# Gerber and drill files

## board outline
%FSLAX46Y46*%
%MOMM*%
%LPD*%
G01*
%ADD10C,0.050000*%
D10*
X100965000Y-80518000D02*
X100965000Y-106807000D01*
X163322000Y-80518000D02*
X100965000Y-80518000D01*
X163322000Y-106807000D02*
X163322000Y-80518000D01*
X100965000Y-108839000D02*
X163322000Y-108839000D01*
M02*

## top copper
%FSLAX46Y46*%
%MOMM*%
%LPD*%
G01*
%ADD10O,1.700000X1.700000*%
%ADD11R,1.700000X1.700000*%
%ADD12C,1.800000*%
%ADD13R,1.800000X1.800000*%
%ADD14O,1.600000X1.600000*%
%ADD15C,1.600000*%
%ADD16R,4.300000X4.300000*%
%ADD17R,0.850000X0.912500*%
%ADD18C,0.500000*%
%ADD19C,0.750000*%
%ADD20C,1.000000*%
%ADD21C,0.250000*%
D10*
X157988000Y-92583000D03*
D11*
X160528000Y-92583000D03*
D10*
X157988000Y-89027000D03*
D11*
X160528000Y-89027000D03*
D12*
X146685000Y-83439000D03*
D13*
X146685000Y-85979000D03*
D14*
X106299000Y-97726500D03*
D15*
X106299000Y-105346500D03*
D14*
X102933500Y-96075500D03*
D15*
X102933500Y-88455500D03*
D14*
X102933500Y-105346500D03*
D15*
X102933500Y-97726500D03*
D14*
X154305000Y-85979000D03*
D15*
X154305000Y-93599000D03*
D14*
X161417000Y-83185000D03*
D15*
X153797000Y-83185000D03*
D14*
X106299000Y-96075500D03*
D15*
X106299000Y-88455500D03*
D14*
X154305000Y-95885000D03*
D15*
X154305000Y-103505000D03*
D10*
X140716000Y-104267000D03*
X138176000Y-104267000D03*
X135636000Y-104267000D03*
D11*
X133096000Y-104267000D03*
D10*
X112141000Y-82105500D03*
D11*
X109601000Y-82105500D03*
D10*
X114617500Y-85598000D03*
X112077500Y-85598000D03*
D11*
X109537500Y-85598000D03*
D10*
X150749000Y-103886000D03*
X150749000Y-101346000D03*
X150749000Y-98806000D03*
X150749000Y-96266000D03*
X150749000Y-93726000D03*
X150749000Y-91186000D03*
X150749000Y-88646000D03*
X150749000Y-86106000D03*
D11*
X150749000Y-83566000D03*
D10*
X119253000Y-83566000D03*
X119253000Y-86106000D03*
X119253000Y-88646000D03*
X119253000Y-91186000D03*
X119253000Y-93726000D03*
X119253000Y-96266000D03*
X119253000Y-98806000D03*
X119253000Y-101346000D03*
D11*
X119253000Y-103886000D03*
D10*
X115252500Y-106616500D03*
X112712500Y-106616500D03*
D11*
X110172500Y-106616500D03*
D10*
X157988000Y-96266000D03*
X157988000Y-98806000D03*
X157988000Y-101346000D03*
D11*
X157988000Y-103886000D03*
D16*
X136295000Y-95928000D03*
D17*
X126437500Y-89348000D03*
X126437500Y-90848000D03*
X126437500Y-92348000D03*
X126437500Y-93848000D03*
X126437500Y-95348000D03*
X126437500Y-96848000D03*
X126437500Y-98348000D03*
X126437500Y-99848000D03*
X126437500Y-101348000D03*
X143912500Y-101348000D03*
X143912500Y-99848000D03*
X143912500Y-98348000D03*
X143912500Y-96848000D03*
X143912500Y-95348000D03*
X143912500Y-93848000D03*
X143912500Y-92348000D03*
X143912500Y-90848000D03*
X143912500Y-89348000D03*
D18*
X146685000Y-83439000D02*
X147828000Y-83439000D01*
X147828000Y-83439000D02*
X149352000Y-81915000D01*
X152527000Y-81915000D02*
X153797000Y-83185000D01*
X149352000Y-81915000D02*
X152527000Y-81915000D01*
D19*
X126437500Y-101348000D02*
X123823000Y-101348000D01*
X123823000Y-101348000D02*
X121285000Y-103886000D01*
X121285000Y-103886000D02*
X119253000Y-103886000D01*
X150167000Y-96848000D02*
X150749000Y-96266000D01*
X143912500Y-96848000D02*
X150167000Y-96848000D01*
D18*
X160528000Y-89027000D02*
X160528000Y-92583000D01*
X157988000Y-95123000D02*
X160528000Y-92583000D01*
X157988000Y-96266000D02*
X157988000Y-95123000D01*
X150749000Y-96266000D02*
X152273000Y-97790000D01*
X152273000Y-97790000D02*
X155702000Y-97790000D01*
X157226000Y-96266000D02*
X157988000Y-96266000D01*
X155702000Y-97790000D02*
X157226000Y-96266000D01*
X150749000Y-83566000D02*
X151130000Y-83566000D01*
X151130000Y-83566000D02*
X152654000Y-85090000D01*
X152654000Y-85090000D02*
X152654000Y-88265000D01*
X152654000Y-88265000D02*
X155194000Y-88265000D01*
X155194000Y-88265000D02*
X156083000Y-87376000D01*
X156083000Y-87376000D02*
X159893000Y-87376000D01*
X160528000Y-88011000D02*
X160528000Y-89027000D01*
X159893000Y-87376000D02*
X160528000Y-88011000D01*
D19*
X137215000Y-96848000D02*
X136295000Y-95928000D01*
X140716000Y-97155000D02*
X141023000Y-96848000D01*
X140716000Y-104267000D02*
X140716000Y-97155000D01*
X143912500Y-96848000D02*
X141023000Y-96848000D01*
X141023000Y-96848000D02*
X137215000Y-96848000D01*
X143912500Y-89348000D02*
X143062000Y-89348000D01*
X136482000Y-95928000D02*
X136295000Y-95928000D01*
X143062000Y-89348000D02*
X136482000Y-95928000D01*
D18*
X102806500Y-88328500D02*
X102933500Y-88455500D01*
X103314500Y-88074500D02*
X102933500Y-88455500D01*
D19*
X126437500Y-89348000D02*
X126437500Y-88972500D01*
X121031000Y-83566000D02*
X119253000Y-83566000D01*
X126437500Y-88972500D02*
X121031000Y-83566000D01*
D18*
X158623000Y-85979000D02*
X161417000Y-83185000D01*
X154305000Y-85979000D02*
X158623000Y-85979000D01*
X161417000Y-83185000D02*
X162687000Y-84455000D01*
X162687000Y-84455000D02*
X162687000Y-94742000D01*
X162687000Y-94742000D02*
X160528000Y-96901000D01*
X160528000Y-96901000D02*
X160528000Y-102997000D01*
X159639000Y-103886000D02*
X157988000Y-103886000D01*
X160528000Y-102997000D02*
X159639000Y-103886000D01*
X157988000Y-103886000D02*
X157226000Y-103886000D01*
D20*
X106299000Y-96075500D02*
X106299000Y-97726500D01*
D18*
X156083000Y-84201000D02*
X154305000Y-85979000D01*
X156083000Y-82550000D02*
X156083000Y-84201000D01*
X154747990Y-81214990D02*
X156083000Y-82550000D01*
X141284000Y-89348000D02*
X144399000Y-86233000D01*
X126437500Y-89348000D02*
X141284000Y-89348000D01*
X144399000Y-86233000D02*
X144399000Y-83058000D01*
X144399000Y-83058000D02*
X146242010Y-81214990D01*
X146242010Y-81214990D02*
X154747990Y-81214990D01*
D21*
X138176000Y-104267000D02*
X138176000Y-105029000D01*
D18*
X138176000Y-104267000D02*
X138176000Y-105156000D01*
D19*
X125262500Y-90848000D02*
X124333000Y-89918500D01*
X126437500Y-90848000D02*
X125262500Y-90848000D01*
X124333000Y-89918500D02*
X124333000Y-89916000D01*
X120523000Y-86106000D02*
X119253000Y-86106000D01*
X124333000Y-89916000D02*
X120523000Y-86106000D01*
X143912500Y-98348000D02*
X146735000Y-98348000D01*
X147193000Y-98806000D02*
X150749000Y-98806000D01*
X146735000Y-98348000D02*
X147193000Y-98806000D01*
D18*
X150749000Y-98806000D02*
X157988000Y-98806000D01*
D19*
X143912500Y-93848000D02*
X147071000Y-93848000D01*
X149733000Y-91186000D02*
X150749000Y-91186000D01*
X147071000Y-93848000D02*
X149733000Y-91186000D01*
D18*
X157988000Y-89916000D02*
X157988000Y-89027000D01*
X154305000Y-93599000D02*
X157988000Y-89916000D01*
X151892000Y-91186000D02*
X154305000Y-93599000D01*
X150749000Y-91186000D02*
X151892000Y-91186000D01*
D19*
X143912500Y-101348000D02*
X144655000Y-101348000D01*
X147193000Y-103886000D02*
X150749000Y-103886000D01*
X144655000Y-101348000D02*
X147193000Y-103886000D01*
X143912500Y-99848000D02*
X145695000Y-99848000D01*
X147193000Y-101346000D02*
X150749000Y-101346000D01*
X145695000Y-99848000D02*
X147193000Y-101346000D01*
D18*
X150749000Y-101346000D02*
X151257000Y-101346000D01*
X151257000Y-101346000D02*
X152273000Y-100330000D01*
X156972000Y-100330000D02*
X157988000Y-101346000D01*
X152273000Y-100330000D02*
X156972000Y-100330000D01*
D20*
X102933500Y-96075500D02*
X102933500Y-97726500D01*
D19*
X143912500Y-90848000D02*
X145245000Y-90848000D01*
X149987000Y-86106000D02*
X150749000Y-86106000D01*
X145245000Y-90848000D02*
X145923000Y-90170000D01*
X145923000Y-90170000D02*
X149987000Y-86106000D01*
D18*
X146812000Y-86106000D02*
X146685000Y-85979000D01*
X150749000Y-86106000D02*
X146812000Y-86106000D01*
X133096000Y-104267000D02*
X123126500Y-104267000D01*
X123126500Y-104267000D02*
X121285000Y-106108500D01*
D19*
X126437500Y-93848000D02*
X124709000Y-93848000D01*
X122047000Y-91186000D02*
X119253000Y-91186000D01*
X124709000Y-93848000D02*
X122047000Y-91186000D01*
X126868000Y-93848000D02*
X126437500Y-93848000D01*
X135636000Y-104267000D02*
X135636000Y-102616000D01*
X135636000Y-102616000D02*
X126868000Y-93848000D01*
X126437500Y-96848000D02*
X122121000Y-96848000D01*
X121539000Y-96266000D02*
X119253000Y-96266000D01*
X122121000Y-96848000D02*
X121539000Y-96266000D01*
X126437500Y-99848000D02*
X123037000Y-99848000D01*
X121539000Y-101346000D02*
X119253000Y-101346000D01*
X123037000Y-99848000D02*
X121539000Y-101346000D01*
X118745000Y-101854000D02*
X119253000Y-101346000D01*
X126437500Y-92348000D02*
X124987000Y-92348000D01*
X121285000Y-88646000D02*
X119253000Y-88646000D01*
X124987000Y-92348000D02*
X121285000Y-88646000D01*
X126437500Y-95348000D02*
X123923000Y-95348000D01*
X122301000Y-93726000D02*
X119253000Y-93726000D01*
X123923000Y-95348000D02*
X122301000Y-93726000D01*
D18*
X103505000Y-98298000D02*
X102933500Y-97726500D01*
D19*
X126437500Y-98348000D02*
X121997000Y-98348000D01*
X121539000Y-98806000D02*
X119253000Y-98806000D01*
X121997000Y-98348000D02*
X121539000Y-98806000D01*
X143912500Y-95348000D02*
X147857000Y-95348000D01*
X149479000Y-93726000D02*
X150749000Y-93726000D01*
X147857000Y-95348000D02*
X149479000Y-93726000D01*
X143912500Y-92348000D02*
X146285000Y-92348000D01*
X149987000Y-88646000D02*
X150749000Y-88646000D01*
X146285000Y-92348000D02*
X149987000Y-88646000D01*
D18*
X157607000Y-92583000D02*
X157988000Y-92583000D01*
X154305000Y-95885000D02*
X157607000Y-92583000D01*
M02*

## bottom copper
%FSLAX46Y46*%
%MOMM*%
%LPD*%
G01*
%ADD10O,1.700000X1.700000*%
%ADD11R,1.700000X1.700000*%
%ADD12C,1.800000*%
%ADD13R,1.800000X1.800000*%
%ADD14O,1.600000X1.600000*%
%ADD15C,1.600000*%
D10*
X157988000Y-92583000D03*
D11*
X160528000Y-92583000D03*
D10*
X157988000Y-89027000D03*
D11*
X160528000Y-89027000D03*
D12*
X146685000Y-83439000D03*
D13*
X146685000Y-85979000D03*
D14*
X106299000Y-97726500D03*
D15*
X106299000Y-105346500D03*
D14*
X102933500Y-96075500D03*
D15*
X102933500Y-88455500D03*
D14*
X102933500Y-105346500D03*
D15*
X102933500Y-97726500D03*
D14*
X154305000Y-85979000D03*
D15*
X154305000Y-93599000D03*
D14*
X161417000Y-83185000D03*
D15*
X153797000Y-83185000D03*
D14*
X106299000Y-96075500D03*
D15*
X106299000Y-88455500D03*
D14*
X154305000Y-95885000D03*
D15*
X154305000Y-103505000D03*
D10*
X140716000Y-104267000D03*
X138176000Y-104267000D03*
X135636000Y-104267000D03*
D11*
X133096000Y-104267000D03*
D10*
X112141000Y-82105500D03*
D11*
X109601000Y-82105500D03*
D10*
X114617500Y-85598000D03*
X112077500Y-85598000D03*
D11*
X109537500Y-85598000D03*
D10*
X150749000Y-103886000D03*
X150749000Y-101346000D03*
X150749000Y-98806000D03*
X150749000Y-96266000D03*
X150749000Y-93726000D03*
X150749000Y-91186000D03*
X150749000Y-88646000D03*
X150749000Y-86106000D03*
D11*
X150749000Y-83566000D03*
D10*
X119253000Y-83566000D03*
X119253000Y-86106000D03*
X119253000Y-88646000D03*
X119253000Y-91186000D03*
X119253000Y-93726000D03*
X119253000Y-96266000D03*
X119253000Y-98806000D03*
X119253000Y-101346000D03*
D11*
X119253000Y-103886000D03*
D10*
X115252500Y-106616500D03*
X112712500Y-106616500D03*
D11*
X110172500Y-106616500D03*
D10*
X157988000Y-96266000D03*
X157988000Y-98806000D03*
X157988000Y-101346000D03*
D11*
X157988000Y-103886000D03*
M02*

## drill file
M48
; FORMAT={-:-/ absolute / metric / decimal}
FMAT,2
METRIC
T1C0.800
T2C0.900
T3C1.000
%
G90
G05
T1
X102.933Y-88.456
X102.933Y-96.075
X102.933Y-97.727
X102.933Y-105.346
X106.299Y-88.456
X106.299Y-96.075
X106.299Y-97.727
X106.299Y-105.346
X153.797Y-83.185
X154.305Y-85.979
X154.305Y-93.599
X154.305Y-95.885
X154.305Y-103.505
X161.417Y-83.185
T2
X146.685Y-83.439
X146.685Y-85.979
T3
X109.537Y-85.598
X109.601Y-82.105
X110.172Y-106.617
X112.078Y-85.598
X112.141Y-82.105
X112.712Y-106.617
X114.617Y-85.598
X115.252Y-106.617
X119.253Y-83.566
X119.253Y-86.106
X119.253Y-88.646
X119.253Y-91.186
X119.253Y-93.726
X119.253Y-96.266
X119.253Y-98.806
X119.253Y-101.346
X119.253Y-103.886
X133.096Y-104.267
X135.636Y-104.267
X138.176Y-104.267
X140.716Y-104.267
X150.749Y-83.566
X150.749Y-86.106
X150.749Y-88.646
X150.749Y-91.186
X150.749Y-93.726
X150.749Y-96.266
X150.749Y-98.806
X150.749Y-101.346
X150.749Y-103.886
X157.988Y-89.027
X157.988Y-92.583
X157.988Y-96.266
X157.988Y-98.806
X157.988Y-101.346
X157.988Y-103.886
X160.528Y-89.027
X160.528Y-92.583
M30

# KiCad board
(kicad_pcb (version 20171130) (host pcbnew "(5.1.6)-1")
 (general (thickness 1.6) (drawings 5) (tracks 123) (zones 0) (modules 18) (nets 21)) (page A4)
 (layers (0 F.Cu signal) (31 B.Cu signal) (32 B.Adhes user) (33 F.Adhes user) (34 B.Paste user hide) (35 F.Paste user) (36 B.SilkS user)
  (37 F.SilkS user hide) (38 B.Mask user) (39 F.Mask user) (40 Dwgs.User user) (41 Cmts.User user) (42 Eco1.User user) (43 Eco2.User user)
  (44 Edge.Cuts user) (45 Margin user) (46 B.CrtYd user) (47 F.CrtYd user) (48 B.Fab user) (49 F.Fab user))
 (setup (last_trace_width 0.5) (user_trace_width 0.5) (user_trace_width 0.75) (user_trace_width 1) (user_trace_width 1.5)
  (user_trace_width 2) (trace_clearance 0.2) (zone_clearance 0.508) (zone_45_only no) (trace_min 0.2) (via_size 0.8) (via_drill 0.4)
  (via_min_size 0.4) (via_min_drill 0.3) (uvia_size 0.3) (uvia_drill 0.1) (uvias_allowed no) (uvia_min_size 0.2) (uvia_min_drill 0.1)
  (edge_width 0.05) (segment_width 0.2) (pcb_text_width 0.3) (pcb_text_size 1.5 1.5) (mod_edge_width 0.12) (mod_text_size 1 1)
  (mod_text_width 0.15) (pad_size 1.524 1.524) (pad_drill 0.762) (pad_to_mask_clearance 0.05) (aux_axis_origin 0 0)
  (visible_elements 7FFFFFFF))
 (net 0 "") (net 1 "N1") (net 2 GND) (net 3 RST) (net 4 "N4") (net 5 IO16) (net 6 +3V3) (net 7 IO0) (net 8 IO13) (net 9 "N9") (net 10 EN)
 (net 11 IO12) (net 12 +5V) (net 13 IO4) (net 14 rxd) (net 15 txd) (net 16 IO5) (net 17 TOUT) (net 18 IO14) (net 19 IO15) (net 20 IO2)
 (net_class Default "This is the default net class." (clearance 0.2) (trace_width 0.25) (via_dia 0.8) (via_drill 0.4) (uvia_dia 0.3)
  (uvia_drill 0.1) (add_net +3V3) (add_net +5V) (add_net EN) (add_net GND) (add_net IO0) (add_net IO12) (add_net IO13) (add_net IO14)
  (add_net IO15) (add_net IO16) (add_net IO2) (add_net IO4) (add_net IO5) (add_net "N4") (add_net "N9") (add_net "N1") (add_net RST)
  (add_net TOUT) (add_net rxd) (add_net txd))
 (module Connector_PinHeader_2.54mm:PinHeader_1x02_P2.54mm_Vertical (layer F.Cu) (at 160.528 92.583 270)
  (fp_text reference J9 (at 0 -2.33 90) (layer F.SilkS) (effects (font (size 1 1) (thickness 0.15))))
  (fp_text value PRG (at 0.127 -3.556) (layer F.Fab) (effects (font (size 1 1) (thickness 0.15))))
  (pad 2 thru_hole oval (at 0 2.54 270) (size 1.7 1.7) (drill 1) (layers *.Cu *.Mask) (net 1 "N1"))
  (pad 1 thru_hole rect (at 0 0 270) (size 1.7 1.7) (drill 1) (layers *.Cu *.Mask) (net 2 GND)))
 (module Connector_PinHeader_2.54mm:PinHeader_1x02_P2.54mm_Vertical (layer F.Cu) (at 160.528 89.027 270)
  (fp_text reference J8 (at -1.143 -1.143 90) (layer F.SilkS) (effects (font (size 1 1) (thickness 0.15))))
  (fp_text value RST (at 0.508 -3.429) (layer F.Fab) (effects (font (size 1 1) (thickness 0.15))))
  (pad 2 thru_hole oval (at 0 2.54 270) (size 1.7 1.7) (drill 1) (layers *.Cu *.Mask) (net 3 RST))
  (pad 1 thru_hole rect (at 0 0 270) (size 1.7 1.7) (drill 1) (layers *.Cu *.Mask) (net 2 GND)))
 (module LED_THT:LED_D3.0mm (layer F.Cu) (at 146.685 85.979 90)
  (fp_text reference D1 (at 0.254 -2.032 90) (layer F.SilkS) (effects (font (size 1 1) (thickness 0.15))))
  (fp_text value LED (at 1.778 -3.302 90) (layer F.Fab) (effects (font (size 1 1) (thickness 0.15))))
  (pad 2 thru_hole circle (at 2.54 0 90) (size 1.8 1.8) (drill 0.9) (layers *.Cu *.Mask) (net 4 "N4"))
  (pad 1 thru_hole rect (at 0 0 90) (size 1.8 1.8) (drill 0.9) (layers *.Cu *.Mask) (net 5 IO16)))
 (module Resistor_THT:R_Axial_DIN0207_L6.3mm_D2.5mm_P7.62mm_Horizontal (layer F.Cu) (at 106.299 105.3465 90)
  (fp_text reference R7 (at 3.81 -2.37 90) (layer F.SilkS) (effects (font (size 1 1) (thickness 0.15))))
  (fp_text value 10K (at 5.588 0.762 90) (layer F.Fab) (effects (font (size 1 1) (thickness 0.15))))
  (pad 2 thru_hole oval (at 7.62 0 90) (size 1.6 1.6) (drill 0.8) (layers *.Cu *.Mask) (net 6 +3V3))
  (pad 1 thru_hole circle (at 0 0 90) (size 1.6 1.6) (drill 0.8) (layers *.Cu *.Mask) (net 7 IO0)))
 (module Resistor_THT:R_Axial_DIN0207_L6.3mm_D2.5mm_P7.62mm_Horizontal (layer F.Cu) (at 102.9335 88.4555 270)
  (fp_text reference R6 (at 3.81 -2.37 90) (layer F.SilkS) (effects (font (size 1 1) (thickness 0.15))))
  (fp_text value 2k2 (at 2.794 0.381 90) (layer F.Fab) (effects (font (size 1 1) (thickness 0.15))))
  (pad 2 thru_hole oval (at 7.62 0 270) (size 1.6 1.6) (drill 0.8) (layers *.Cu *.Mask) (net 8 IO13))
  (pad 1 thru_hole circle (at 0 0 270) (size 1.6 1.6) (drill 0.8) (layers *.Cu *.Mask) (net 2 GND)))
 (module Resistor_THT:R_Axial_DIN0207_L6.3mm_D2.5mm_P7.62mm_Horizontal (layer F.Cu) (at 102.9335 97.7265 270)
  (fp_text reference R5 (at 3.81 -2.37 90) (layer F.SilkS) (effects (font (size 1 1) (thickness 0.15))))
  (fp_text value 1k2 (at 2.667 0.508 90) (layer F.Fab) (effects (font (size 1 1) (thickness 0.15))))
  (pad 2 thru_hole oval (at 7.62 0 270) (size 1.6 1.6) (drill 0.8) (layers *.Cu *.Mask) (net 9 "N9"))
  (pad 1 thru_hole circle (at 0 0 270) (size 1.6 1.6) (drill 0.8) (layers *.Cu *.Mask) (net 8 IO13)))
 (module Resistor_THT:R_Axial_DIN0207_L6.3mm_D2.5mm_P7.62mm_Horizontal (layer F.Cu) (at 154.305 93.599 90)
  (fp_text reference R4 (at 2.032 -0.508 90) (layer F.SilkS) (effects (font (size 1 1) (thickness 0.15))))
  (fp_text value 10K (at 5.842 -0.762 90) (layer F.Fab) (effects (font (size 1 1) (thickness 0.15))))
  (pad 2 thru_hole oval (at 7.62 0 90) (size 1.6 1.6) (drill 0.8) (layers *.Cu *.Mask) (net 6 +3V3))
  (pad 1 thru_hole circle (at 0 0 90) (size 1.6 1.6) (drill 0.8) (layers *.Cu *.Mask) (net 3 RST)))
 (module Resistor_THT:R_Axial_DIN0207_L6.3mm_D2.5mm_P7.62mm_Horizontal (layer F.Cu) (at 153.797 83.185)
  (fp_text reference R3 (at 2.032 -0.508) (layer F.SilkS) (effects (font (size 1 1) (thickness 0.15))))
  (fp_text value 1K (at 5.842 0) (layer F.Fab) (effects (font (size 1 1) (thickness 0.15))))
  (pad 2 thru_hole oval (at 7.62 0) (size 1.6 1.6) (drill 0.8) (layers *.Cu *.Mask) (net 6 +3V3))
  (pad 1 thru_hole circle (at 0 0) (size 1.6 1.6) (drill 0.8) (layers *.Cu *.Mask) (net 4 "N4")))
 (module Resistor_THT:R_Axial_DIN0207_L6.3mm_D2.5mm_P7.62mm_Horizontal (layer F.Cu) (at 106.299 88.4555 270)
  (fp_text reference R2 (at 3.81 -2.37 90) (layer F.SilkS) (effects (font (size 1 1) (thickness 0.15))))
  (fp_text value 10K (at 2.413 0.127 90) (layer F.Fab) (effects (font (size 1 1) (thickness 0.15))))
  (pad 2 thru_hole oval (at 7.62 0 270) (size 1.6 1.6) (drill 0.8) (layers *.Cu *.Mask) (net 6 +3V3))
  (pad 1 thru_hole circle (at 0 0 270) (size 1.6 1.6) (drill 0.8) (layers *.Cu *.Mask) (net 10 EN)))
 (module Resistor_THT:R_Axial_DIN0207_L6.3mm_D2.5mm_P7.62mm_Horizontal (layer F.Cu) (at 154.305 103.505 90)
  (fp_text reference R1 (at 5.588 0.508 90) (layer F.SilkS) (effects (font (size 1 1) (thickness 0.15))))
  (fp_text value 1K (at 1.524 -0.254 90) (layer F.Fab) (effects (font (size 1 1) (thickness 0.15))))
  (pad 2 thru_hole oval (at 7.62 0 90) (size 1.6 1.6) (drill 0.8) (layers *.Cu *.Mask) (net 1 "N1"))
  (pad 1 thru_hole circle (at 0 0 90) (size 1.6 1.6) (drill 0.8) (layers *.Cu *.Mask) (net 7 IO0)))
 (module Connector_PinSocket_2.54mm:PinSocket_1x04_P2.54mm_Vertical (layer F.Cu) (at 133.096 104.267 90)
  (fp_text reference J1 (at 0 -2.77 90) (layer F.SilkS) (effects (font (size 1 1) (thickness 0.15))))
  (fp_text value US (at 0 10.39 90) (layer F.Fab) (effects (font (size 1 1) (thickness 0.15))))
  (pad 4 thru_hole oval (at 0 7.62 90) (size 1.7 1.7) (drill 1) (layers *.Cu *.Mask) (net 2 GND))
  (pad 3 thru_hole oval (at 0 5.08 90) (size 1.7 1.7) (drill 1) (layers *.Cu *.Mask) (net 9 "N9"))
  (pad 2 thru_hole oval (at 0 2.54 90) (size 1.7 1.7) (drill 1) (layers *.Cu *.Mask) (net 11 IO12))
  (pad 1 thru_hole rect (at 0 0 90) (size 1.7 1.7) (drill 1) (layers *.Cu *.Mask) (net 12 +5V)))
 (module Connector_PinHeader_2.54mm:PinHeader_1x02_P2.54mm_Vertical (layer F.Cu) (at 109.601 82.1055 90)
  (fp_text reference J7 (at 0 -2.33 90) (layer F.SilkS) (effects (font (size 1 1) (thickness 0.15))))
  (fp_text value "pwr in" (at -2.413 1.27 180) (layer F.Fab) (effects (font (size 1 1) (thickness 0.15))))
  (pad 2 thru_hole oval (at 0 2.54 90) (size 1.7 1.7) (drill 1) (layers *.Cu *.Mask) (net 2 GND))
  (pad 1 thru_hole rect (at 0 0 90) (size 1.7 1.7) (drill 1) (layers *.Cu *.Mask) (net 12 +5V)))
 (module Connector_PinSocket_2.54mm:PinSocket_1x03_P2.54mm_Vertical (layer F.Cu) (at 109.5375 85.598 90)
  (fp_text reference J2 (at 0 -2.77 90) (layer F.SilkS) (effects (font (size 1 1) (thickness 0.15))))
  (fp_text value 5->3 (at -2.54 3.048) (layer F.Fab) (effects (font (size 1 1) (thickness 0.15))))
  (pad 3 thru_hole oval (at 0 5.08 90) (size 1.7 1.7) (drill 1) (layers *.Cu *.Mask) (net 2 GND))
  (pad 2 thru_hole oval (at 0 2.54 90) (size 1.7 1.7) (drill 1) (layers *.Cu *.Mask) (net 6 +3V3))
  (pad 1 thru_hole rect (at 0 0 90) (size 1.7 1.7) (drill 1) (layers *.Cu *.Mask) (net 12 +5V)))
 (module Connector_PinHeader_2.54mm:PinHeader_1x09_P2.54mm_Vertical (layer F.Cu) (at 150.749 83.566)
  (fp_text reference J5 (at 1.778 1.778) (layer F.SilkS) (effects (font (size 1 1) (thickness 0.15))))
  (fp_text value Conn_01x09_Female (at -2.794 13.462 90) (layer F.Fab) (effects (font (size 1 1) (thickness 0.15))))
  (pad 9 thru_hole oval (at 0 20.32) (size 1.7 1.7) (drill 1) (layers *.Cu *.Mask) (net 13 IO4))
  (pad 8 thru_hole oval (at 0 17.78) (size 1.7 1.7) (drill 1) (layers *.Cu *.Mask) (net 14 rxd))
  (pad 7 thru_hole oval (at 0 15.24) (size 1.7 1.7) (drill 1) (layers *.Cu *.Mask) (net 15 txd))
  (pad 6 thru_hole oval (at 0 12.7) (size 1.7 1.7) (drill 1) (layers *.Cu *.Mask) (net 2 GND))
  (pad 5 thru_hole oval (at 0 10.16) (size 1.7 1.7) (drill 1) (layers *.Cu *.Mask) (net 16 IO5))
  (pad 4 thru_hole oval (at 0 7.62) (size 1.7 1.7) (drill 1) (layers *.Cu *.Mask) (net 3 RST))
  (pad 3 thru_hole oval (at 0 5.08) (size 1.7 1.7) (drill 1) (layers *.Cu *.Mask) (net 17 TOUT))
  (pad 2 thru_hole oval (at 0 2.54) (size 1.7 1.7) (drill 1) (layers *.Cu *.Mask) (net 5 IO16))
  (pad 1 thru_hole rect (at 0 0) (size 1.7 1.7) (drill 1) (layers *.Cu *.Mask) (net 2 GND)))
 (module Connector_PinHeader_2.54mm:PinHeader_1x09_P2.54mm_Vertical (layer F.Cu) (at 119.253 103.886 180)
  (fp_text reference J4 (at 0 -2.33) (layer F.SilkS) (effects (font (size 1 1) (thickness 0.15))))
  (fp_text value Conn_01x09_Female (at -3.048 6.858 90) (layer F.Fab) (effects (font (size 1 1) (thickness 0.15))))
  (pad 9 thru_hole oval (at 0 20.32 180) (size 1.7 1.7) (drill 1) (layers *.Cu *.Mask) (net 6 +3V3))
  (pad 8 thru_hole oval (at 0 17.78 180) (size 1.7 1.7) (drill 1) (layers *.Cu *.Mask) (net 10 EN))
  (pad 7 thru_hole oval (at 0 15.24 180) (size 1.7 1.7) (drill 1) (layers *.Cu *.Mask) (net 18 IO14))
  (pad 6 thru_hole oval (at 0 12.7 180) (size 1.7 1.7) (drill 1) (layers *.Cu *.Mask) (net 11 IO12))
  (pad 5 thru_hole oval (at 0 10.16 180) (size 1.7 1.7) (drill 1) (layers *.Cu *.Mask) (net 8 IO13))
  (pad 4 thru_hole oval (at 0 7.62 180) (size 1.7 1.7) (drill 1) (layers *.Cu *.Mask) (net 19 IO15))
  (pad 3 thru_hole oval (at 0 5.08 180) (size 1.7 1.7) (drill 1) (layers *.Cu *.Mask) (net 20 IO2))
  (pad 2 thru_hole oval (at 0 2.54 180) (size 1.7 1.7) (drill 1) (layers *.Cu *.Mask) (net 7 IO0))
  (pad 1 thru_hole rect (at 0 0 180) (size 1.7 1.7) (drill 1) (layers *.Cu *.Mask) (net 2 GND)))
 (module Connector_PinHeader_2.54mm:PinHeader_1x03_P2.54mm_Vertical (layer F.Cu) (at 110.1725 106.6165 90)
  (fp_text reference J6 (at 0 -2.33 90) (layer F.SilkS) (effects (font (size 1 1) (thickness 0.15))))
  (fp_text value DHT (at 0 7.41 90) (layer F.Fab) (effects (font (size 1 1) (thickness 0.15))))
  (pad 3 thru_hole oval (at 0 5.08 90) (size 1.7 1.7) (drill 1) (layers *.Cu *.Mask) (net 18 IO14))
  (pad 2 thru_hole oval (at 0 2.54 90) (size 1.7 1.7) (drill 1) (layers *.Cu *.Mask) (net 2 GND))
  (pad 1 thru_hole rect (at 0 0 90) (size 1.7 1.7) (drill 1) (layers *.Cu *.Mask) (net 6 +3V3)))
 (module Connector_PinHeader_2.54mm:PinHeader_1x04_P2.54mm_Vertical (layer F.Cu) (at 157.988 103.886 180)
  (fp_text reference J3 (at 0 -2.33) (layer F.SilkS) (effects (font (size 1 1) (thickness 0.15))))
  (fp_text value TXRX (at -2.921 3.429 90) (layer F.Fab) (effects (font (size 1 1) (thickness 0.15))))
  (pad 4 thru_hole oval (at 0 7.62 180) (size 1.7 1.7) (drill 1) (layers *.Cu *.Mask) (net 2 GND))
  (pad 3 thru_hole oval (at 0 5.08 180) (size 1.7 1.7) (drill 1) (layers *.Cu *.Mask) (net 15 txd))
  (pad 2 thru_hole oval (at 0 2.54 180) (size 1.7 1.7) (drill 1) (layers *.Cu *.Mask) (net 14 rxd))
  (pad 1 thru_hole rect (at 0 0 180) (size 1.7 1.7) (drill 1) (layers *.Cu *.Mask) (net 6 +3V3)))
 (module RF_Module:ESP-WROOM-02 (layer F.Cu) (at 135.175 95.348)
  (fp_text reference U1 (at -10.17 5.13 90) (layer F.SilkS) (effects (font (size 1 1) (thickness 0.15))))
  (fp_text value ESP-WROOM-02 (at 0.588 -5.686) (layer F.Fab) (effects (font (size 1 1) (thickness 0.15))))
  (pad 19 smd rect (at 1.12 0.58) (size 4.3 4.3) (layers F.Cu F.Paste F.Mask) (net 2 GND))
  (pad 1 smd rect (at -8.7375 -6) (size 0.85 0.9125) (layers F.Cu F.Paste F.Mask) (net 6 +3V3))
  (pad 2 smd rect (at -8.7375 -4.5) (size 0.85 0.9125) (layers F.Cu F.Paste F.Mask) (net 10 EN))
  (pad 3 smd rect (at -8.7375 -3) (size 0.85 0.9125) (layers F.Cu F.Paste F.Mask) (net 18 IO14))
  (pad 4 smd rect (at -8.7375 -1.5) (size 0.85 0.9125) (layers F.Cu F.Paste F.Mask) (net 11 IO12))
  (pad 5 smd rect (at -8.7375 0) (size 0.85 0.9125) (layers F.Cu F.Paste F.Mask) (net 8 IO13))
  (pad 6 smd rect (at -8.7375 1.5) (size 0.85 0.9125) (layers F.Cu F.Paste F.Mask) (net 19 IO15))
  (pad 7 smd rect (at -8.7375 3) (size 0.85 0.9125) (layers F.Cu F.Paste F.Mask) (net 20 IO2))
  (pad 8 smd rect (at -8.7375 4.5) (size 0.85 0.9125) (layers F.Cu F.Paste F.Mask) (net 7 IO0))
  (pad 9 smd rect (at -8.7375 6) (size 0.85 0.9125) (layers F.Cu F.Paste F.Mask) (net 2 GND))
  (pad 10 smd rect (at 8.7375 6) (size 0.85 0.9125) (layers F.Cu F.Paste F.Mask) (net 13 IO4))
  (pad 11 smd rect (at 8.7375 4.5) (size 0.85 0.9125) (layers F.Cu F.Paste F.Mask) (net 14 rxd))
  (pad 12 smd rect (at 8.7375 3) (size 0.85 0.9125) (layers F.Cu F.Paste F.Mask) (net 15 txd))
  (pad 13 smd rect (at 8.7375 1.5) (size 0.85 0.9125) (layers F.Cu F.Paste F.Mask) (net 2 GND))
  (pad 14 smd rect (at 8.7375 0) (size 0.85 0.9125) (layers F.Cu F.Paste F.Mask) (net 16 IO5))
  (pad 15 smd rect (at 8.7375 -1.5) (size 0.85 0.9125) (layers F.Cu F.Paste F.Mask) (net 3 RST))
  (pad 16 smd rect (at 8.7375 -3) (size 0.85 0.9125) (layers F.Cu F.Paste F.Mask) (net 17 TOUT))
  (pad 17 smd rect (at 8.7375 -4.5) (size 0.85 0.9125) (layers F.Cu F.Paste F.Mask) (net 5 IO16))
  (pad 18 smd rect (at 8.7375 -6) (size 0.85 0.9125) (layers F.Cu F.Paste F.Mask) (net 2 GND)))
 (gr_line (start 100.965 80.518) (end 100.965 106.807) (layer Edge.Cuts) (width 0.05))
 (gr_line (start 163.322 80.518) (end 100.965 80.518) (layer Edge.Cuts) (width 0.05))
 (gr_line (start 163.322 106.807) (end 163.322 80.518) (layer Edge.Cuts) (width 0.05))
 (gr_line (start 100.965 108.839) (end 163.322 108.839) (layer Edge.Cuts) (width 0.05))
 (segment (start 146.685 83.439) (end 147.828 83.439) (width 0.5) (layer F.Cu) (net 4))
 (segment (start 147.828 83.439) (end 149.352 81.915) (width 0.5) (layer F.Cu) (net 4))
 (segment (start 152.527 81.915) (end 153.797 83.185) (width 0.5) (layer F.Cu) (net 4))
 (segment (start 149.352 81.915) (end 152.527 81.915) (width 0.5) (layer F.Cu) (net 4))
 (segment (start 126.4375 101.348) (end 123.823 101.348) (width 0.75) (layer F.Cu) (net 2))
 (segment (start 123.823 101.348) (end 121.285 103.886) (width 0.75) (layer F.Cu) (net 2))
 (segment (start 121.285 103.886) (end 119.253 103.886) (width 0.75) (layer F.Cu) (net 2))
 (segment (start 150.167 96.848) (end 150.749 96.266) (width 0.75) (layer F.Cu) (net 2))
 (segment (start 143.9125 96.848) (end 150.167 96.848) (width 0.75) (layer F.Cu) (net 2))
 (segment (start 160.528 89.027) (end 160.528 92.583) (width 0.5) (layer F.Cu) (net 2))
 (segment (start 157.988 95.123) (end 160.528 92.583) (width 0.5) (layer F.Cu) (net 2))
 (segment (start 157.988 96.266) (end 157.988 95.123) (width 0.5) (layer F.Cu) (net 2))
 (segment (start 150.749 96.266) (end 152.273 97.79) (width 0.5) (layer F.Cu) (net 2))
 (segment (start 152.273 97.79) (end 155.702 97.79) (width 0.5) (layer F.Cu) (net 2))
 (segment (start 157.226 96.266) (end 157.988 96.266) (width 0.5) (layer F.Cu) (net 2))
 (segment (start 155.702 97.79) (end 157.226 96.266) (width 0.5) (layer F.Cu) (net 2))
 (segment (start 150.749 83.566) (end 151.13 83.566) (width 0.5) (layer F.Cu) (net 2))
 (segment (start 151.13 83.566) (end 152.654 85.09) (width 0.5) (layer F.Cu) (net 2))
 (segment (start 152.654 85.09) (end 152.654 88.265) (width 0.5) (layer F.Cu) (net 2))
 (segment (start 152.654 88.265) (end 155.194 88.265) (width 0.5) (layer F.Cu) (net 2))
 (segment (start 155.194 88.265) (end 156.083 87.376) (width 0.5) (layer F.Cu) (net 2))
 (segment (start 156.083 87.376) (end 159.893 87.376) (width 0.5) (layer F.Cu) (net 2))
 (segment (start 160.528 88.011) (end 160.528 89.027) (width 0.5) (layer F.Cu) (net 2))
 (segment (start 159.893 87.376) (end 160.528 88.011) (width 0.5) (layer F.Cu) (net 2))
 (segment (start 137.215 96.848) (end 136.295 95.928) (width 0.75) (layer F.Cu) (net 2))
 (segment (start 140.716 97.155) (end 141.023 96.848) (width 0.75) (layer F.Cu) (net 2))
 (segment (start 140.716 104.267) (end 140.716 97.155) (width 0.75) (layer F.Cu) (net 2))
 (segment (start 143.9125 96.848) (end 141.023 96.848) (width 0.75) (layer F.Cu) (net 2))
 (segment (start 141.023 96.848) (end 137.215 96.848) (width 0.75) (layer F.Cu) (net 2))
 (segment (start 143.9125 89.348) (end 143.062 89.348) (width 0.75) (layer F.Cu) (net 2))
 (segment (start 136.482 95.928) (end 136.295 95.928) (width 0.75) (layer F.Cu) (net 2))
 (segment (start 143.062 89.348) (end 136.482 95.928) (width 0.75) (layer F.Cu) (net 2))
 (segment (start 102.8065 88.3285) (end 102.9335 88.4555) (width 0.5) (layer F.Cu) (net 2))
 (segment (start 103.3145 88.0745) (end 102.9335 88.4555) (width 0.5) (layer F.Cu) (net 2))
 (segment (start 126.4375 89.348) (end 126.4375 88.9725) (width 0.75) (layer F.Cu) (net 6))
 (segment (start 121.031 83.566) (end 119.253 83.566) (width 0.75) (layer F.Cu) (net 6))
 (segment (start 126.4375 88.9725) (end 121.031 83.566) (width 0.75) (layer F.Cu) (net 6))
 (segment (start 158.623 85.979) (end 161.417 83.185) (width 0.5) (layer F.Cu) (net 6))
 (segment (start 154.305 85.979) (end 158.623 85.979) (width 0.5) (layer F.Cu) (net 6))
 (segment (start 161.417 83.185) (end 162.687 84.455) (width 0.5) (layer F.Cu) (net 6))
 (segment (start 162.687 84.455) (end 162.687 94.742) (width 0.5) (layer F.Cu) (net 6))
 (segment (start 162.687 94.742) (end 160.528 96.901) (width 0.5) (layer F.Cu) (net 6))
 (segment (start 160.528 96.901) (end 160.528 102.997) (width 0.5) (layer F.Cu) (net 6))
 (segment (start 159.639 103.886) (end 157.988 103.886) (width 0.5) (layer F.Cu) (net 6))
 (segment (start 160.528 102.997) (end 159.639 103.886) (width 0.5) (layer F.Cu) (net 6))
 (segment (start 157.988 103.886) (end 157.226 103.886) (width 0.5) (layer F.Cu) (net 6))
 (segment (start 106.299 96.0755) (end 106.299 97.7265) (width 1) (layer F.Cu) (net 6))
 (segment (start 156.083 84.201) (end 154.305 85.979) (width 0.5) (layer F.Cu) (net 6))
 (segment (start 156.083 82.55) (end 156.083 84.201) (width 0.5) (layer F.Cu) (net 6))
 (segment (start 154.74799 81.21499) (end 156.083 82.55) (width 0.5) (layer F.Cu) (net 6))
 (segment (start 141.284 89.348) (end 144.399 86.233) (width 0.5) (layer F.Cu) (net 6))
 (segment (start 126.4375 89.348) (end 141.284 89.348) (width 0.5) (layer F.Cu) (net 6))
 (segment (start 144.399 86.233) (end 144.399 83.058) (width 0.5) (layer F.Cu) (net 6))
 (segment (start 144.399 83.058) (end 146.24201 81.21499) (width 0.5) (layer F.Cu) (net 6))
 (segment (start 146.24201 81.21499) (end 154.74799 81.21499) (width 0.5) (layer F.Cu) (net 6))
 (segment (start 138.176 104.267) (end 138.176 105.029) (width 0.25) (layer F.Cu) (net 9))
 (segment (start 138.176 104.267) (end 138.176 105.156) (width 0.5) (layer F.Cu) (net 9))
 (segment (start 125.2625 90.848) (end 124.333 89.9185) (width 0.75) (layer F.Cu) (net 10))
 (segment (start 126.4375 90.848) (end 125.2625 90.848) (width 0.75) (layer F.Cu) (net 10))
 (segment (start 124.333 89.9185) (end 124.333 89.916) (width 0.75) (layer F.Cu) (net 10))
 (segment (start 120.523 86.106) (end 119.253 86.106) (width 0.75) (layer F.Cu) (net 10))
 (segment (start 124.333 89.916) (end 120.523 86.106) (width 0.75) (layer F.Cu) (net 10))
 (segment (start 143.9125 98.348) (end 146.735 98.348) (width 0.75) (layer F.Cu) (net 15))
 (segment (start 147.193 98.806) (end 150.749 98.806) (width 0.75) (layer F.Cu) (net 15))
 (segment (start 146.735 98.348) (end 147.193 98.806) (width 0.75) (layer F.Cu) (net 15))
 (segment (start 150.749 98.806) (end 157.988 98.806) (width 0.5) (layer F.Cu) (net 15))
 (segment (start 143.9125 93.848) (end 147.071 93.848) (width 0.75) (layer F.Cu) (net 3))
 (segment (start 149.733 91.186) (end 150.749 91.186) (width 0.75) (layer F.Cu) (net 3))
 (segment (start 147.071 93.848) (end 149.733 91.186) (width 0.75) (layer F.Cu) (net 3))
 (segment (start 157.988 89.916) (end 157.988 89.027) (width 0.5) (layer F.Cu) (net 3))
 (segment (start 154.305 93.599) (end 157.988 89.916) (width 0.5) (layer F.Cu) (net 3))
 (segment (start 151.892 91.186) (end 154.305 93.599) (width 0.5) (layer F.Cu) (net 3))
 (segment (start 150.749 91.186) (end 151.892 91.186) (width 0.5) (layer F.Cu) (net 3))
 (segment (start 143.9125 101.348) (end 144.655 101.348) (width 0.75) (layer F.Cu) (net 13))
 (segment (start 147.193 103.886) (end 150.749 103.886) (width 0.75) (layer F.Cu) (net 13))
 (segment (start 144.655 101.348) (end 147.193 103.886) (width 0.75) (layer F.Cu) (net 13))
 (segment (start 143.9125 99.848) (end 145.695 99.848) (width 0.75) (layer F.Cu) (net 14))
 (segment (start 147.193 101.346) (end 150.749 101.346) (width 0.75) (layer F.Cu) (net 14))
 (segment (start 145.695 99.848) (end 147.193 101.346) (width 0.75) (layer F.Cu) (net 14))
 (segment (start 150.749 101.346) (end 151.257 101.346) (width 0.5) (layer F.Cu) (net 14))
 (segment (start 151.257 101.346) (end 152.273 100.33) (width 0.5) (layer F.Cu) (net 14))
 (segment (start 156.972 100.33) (end 157.988 101.346) (width 0.5) (layer F.Cu) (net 14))
 (segment (start 152.273 100.33) (end 156.972 100.33) (width 0.5) (layer F.Cu) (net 14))
 (segment (start 102.9335 96.0755) (end 102.9335 97.7265) (width 1) (layer F.Cu) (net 8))
 (segment (start 143.9125 90.848) (end 145.245 90.848) (width 0.75) (layer F.Cu) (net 5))
 (segment (start 149.987 86.106) (end 150.749 86.106) (width 0.75) (layer F.Cu) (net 5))
 (segment (start 145.245 90.848) (end 145.923 90.17) (width 0.75) (layer F.Cu) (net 5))
 (segment (start 145.923 90.17) (end 149.987 86.106) (width 0.75) (layer F.Cu) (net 5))
 (segment (start 146.812 86.106) (end 146.685 85.979) (width 0.5) (layer F.Cu) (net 5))
 (segment (start 150.749 86.106) (end 146.812 86.106) (width 0.5) (layer F.Cu) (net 5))
 (segment (start 133.096 104.267) (end 123.1265 104.267) (width 0.5) (layer F.Cu) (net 12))
 (segment (start 123.1265 104.267) (end 121.285 106.1085) (width 0.5) (layer F.Cu) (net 12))
 (segment (start 126.4375 93.848) (end 124.709 93.848) (width 0.75) (layer F.Cu) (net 11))
 (segment (start 122.047 91.186) (end 119.253 91.186) (width 0.75) (layer F.Cu) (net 11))
 (segment (start 124.709 93.848) (end 122.047 91.186) (width 0.75) (layer F.Cu) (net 11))
 (segment (start 126.868 93.848) (end 126.4375 93.848) (width 0.75) (layer F.Cu) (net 11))
 (segment (start 135.636 104.267) (end 135.636 102.616) (width 0.75) (layer F.Cu) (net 11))
 (segment (start 135.636 102.616) (end 126.868 93.848) (width 0.75) (layer F.Cu) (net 11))
 (segment (start 126.4375 96.848) (end 122.121 96.848) (width 0.75) (layer F.Cu) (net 19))
 (segment (start 121.539 96.266) (end 119.253 96.266) (width 0.75) (layer F.Cu) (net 19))
 (segment (start 122.121 96.848) (end 121.539 96.266) (width 0.75) (layer F.Cu) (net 19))
 (segment (start 126.4375 99.848) (end 123.037 99.848) (width 0.75) (layer F.Cu) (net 7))
 (segment (start 121.539 101.346) (end 119.253 101.346) (width 0.75) (layer F.Cu) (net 7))
 (segment (start 123.037 99.848) (end 121.539 101.346) (width 0.75) (layer F.Cu) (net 7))
 (segment (start 118.745 101.854) (end 119.253 101.346) (width 0.75) (layer F.Cu) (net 7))
 (segment (start 126.4375 92.348) (end 124.987 92.348) (width 0.75) (layer F.Cu) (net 18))
 (segment (start 121.285 88.646) (end 119.253 88.646) (width 0.75) (layer F.Cu) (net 18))
 (segment (start 124.987 92.348) (end 121.285 88.646) (width 0.75) (layer F.Cu) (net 18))
 (segment (start 126.4375 95.348) (end 123.923 95.348) (width 0.75) (layer F.Cu) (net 8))
 (segment (start 122.301 93.726) (end 119.253 93.726) (width 0.75) (layer F.Cu) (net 8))
 (segment (start 123.923 95.348) (end 122.301 93.726) (width 0.75) (layer F.Cu) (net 8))
 (segment (start 103.505 98.298) (end 102.9335 97.7265) (width 0.5) (layer F.Cu) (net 8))
 (segment (start 126.4375 98.348) (end 121.997 98.348) (width 0.75) (layer F.Cu) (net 20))
 (segment (start 121.539 98.806) (end 119.253 98.806) (width 0.75) (layer F.Cu) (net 20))
 (segment (start 121.997 98.348) (end 121.539 98.806) (width 0.75) (layer F.Cu) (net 20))
 (segment (start 143.9125 95.348) (end 147.857 95.348) (width 0.75) (layer F.Cu) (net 16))
 (segment (start 149.479 93.726) (end 150.749 93.726) (width 0.75) (layer F.Cu) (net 16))
 (segment (start 147.857 95.348) (end 149.479 93.726) (width 0.75) (layer F.Cu) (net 16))
 (segment (start 143.9125 92.348) (end 146.285 92.348) (width 0.75) (layer F.Cu) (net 17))
 (segment (start 149.987 88.646) (end 150.749 88.646) (width 0.75) (layer F.Cu) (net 17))
 (segment (start 146.285 92.348) (end 149.987 88.646) (width 0.75) (layer F.Cu) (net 17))
 (segment (start 157.607 92.583) (end 157.988 92.583) (width 0.5) (layer F.Cu) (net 1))
 (segment (start 154.305 95.885) (end 157.607 92.583) (width 0.5) (layer F.Cu) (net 1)))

